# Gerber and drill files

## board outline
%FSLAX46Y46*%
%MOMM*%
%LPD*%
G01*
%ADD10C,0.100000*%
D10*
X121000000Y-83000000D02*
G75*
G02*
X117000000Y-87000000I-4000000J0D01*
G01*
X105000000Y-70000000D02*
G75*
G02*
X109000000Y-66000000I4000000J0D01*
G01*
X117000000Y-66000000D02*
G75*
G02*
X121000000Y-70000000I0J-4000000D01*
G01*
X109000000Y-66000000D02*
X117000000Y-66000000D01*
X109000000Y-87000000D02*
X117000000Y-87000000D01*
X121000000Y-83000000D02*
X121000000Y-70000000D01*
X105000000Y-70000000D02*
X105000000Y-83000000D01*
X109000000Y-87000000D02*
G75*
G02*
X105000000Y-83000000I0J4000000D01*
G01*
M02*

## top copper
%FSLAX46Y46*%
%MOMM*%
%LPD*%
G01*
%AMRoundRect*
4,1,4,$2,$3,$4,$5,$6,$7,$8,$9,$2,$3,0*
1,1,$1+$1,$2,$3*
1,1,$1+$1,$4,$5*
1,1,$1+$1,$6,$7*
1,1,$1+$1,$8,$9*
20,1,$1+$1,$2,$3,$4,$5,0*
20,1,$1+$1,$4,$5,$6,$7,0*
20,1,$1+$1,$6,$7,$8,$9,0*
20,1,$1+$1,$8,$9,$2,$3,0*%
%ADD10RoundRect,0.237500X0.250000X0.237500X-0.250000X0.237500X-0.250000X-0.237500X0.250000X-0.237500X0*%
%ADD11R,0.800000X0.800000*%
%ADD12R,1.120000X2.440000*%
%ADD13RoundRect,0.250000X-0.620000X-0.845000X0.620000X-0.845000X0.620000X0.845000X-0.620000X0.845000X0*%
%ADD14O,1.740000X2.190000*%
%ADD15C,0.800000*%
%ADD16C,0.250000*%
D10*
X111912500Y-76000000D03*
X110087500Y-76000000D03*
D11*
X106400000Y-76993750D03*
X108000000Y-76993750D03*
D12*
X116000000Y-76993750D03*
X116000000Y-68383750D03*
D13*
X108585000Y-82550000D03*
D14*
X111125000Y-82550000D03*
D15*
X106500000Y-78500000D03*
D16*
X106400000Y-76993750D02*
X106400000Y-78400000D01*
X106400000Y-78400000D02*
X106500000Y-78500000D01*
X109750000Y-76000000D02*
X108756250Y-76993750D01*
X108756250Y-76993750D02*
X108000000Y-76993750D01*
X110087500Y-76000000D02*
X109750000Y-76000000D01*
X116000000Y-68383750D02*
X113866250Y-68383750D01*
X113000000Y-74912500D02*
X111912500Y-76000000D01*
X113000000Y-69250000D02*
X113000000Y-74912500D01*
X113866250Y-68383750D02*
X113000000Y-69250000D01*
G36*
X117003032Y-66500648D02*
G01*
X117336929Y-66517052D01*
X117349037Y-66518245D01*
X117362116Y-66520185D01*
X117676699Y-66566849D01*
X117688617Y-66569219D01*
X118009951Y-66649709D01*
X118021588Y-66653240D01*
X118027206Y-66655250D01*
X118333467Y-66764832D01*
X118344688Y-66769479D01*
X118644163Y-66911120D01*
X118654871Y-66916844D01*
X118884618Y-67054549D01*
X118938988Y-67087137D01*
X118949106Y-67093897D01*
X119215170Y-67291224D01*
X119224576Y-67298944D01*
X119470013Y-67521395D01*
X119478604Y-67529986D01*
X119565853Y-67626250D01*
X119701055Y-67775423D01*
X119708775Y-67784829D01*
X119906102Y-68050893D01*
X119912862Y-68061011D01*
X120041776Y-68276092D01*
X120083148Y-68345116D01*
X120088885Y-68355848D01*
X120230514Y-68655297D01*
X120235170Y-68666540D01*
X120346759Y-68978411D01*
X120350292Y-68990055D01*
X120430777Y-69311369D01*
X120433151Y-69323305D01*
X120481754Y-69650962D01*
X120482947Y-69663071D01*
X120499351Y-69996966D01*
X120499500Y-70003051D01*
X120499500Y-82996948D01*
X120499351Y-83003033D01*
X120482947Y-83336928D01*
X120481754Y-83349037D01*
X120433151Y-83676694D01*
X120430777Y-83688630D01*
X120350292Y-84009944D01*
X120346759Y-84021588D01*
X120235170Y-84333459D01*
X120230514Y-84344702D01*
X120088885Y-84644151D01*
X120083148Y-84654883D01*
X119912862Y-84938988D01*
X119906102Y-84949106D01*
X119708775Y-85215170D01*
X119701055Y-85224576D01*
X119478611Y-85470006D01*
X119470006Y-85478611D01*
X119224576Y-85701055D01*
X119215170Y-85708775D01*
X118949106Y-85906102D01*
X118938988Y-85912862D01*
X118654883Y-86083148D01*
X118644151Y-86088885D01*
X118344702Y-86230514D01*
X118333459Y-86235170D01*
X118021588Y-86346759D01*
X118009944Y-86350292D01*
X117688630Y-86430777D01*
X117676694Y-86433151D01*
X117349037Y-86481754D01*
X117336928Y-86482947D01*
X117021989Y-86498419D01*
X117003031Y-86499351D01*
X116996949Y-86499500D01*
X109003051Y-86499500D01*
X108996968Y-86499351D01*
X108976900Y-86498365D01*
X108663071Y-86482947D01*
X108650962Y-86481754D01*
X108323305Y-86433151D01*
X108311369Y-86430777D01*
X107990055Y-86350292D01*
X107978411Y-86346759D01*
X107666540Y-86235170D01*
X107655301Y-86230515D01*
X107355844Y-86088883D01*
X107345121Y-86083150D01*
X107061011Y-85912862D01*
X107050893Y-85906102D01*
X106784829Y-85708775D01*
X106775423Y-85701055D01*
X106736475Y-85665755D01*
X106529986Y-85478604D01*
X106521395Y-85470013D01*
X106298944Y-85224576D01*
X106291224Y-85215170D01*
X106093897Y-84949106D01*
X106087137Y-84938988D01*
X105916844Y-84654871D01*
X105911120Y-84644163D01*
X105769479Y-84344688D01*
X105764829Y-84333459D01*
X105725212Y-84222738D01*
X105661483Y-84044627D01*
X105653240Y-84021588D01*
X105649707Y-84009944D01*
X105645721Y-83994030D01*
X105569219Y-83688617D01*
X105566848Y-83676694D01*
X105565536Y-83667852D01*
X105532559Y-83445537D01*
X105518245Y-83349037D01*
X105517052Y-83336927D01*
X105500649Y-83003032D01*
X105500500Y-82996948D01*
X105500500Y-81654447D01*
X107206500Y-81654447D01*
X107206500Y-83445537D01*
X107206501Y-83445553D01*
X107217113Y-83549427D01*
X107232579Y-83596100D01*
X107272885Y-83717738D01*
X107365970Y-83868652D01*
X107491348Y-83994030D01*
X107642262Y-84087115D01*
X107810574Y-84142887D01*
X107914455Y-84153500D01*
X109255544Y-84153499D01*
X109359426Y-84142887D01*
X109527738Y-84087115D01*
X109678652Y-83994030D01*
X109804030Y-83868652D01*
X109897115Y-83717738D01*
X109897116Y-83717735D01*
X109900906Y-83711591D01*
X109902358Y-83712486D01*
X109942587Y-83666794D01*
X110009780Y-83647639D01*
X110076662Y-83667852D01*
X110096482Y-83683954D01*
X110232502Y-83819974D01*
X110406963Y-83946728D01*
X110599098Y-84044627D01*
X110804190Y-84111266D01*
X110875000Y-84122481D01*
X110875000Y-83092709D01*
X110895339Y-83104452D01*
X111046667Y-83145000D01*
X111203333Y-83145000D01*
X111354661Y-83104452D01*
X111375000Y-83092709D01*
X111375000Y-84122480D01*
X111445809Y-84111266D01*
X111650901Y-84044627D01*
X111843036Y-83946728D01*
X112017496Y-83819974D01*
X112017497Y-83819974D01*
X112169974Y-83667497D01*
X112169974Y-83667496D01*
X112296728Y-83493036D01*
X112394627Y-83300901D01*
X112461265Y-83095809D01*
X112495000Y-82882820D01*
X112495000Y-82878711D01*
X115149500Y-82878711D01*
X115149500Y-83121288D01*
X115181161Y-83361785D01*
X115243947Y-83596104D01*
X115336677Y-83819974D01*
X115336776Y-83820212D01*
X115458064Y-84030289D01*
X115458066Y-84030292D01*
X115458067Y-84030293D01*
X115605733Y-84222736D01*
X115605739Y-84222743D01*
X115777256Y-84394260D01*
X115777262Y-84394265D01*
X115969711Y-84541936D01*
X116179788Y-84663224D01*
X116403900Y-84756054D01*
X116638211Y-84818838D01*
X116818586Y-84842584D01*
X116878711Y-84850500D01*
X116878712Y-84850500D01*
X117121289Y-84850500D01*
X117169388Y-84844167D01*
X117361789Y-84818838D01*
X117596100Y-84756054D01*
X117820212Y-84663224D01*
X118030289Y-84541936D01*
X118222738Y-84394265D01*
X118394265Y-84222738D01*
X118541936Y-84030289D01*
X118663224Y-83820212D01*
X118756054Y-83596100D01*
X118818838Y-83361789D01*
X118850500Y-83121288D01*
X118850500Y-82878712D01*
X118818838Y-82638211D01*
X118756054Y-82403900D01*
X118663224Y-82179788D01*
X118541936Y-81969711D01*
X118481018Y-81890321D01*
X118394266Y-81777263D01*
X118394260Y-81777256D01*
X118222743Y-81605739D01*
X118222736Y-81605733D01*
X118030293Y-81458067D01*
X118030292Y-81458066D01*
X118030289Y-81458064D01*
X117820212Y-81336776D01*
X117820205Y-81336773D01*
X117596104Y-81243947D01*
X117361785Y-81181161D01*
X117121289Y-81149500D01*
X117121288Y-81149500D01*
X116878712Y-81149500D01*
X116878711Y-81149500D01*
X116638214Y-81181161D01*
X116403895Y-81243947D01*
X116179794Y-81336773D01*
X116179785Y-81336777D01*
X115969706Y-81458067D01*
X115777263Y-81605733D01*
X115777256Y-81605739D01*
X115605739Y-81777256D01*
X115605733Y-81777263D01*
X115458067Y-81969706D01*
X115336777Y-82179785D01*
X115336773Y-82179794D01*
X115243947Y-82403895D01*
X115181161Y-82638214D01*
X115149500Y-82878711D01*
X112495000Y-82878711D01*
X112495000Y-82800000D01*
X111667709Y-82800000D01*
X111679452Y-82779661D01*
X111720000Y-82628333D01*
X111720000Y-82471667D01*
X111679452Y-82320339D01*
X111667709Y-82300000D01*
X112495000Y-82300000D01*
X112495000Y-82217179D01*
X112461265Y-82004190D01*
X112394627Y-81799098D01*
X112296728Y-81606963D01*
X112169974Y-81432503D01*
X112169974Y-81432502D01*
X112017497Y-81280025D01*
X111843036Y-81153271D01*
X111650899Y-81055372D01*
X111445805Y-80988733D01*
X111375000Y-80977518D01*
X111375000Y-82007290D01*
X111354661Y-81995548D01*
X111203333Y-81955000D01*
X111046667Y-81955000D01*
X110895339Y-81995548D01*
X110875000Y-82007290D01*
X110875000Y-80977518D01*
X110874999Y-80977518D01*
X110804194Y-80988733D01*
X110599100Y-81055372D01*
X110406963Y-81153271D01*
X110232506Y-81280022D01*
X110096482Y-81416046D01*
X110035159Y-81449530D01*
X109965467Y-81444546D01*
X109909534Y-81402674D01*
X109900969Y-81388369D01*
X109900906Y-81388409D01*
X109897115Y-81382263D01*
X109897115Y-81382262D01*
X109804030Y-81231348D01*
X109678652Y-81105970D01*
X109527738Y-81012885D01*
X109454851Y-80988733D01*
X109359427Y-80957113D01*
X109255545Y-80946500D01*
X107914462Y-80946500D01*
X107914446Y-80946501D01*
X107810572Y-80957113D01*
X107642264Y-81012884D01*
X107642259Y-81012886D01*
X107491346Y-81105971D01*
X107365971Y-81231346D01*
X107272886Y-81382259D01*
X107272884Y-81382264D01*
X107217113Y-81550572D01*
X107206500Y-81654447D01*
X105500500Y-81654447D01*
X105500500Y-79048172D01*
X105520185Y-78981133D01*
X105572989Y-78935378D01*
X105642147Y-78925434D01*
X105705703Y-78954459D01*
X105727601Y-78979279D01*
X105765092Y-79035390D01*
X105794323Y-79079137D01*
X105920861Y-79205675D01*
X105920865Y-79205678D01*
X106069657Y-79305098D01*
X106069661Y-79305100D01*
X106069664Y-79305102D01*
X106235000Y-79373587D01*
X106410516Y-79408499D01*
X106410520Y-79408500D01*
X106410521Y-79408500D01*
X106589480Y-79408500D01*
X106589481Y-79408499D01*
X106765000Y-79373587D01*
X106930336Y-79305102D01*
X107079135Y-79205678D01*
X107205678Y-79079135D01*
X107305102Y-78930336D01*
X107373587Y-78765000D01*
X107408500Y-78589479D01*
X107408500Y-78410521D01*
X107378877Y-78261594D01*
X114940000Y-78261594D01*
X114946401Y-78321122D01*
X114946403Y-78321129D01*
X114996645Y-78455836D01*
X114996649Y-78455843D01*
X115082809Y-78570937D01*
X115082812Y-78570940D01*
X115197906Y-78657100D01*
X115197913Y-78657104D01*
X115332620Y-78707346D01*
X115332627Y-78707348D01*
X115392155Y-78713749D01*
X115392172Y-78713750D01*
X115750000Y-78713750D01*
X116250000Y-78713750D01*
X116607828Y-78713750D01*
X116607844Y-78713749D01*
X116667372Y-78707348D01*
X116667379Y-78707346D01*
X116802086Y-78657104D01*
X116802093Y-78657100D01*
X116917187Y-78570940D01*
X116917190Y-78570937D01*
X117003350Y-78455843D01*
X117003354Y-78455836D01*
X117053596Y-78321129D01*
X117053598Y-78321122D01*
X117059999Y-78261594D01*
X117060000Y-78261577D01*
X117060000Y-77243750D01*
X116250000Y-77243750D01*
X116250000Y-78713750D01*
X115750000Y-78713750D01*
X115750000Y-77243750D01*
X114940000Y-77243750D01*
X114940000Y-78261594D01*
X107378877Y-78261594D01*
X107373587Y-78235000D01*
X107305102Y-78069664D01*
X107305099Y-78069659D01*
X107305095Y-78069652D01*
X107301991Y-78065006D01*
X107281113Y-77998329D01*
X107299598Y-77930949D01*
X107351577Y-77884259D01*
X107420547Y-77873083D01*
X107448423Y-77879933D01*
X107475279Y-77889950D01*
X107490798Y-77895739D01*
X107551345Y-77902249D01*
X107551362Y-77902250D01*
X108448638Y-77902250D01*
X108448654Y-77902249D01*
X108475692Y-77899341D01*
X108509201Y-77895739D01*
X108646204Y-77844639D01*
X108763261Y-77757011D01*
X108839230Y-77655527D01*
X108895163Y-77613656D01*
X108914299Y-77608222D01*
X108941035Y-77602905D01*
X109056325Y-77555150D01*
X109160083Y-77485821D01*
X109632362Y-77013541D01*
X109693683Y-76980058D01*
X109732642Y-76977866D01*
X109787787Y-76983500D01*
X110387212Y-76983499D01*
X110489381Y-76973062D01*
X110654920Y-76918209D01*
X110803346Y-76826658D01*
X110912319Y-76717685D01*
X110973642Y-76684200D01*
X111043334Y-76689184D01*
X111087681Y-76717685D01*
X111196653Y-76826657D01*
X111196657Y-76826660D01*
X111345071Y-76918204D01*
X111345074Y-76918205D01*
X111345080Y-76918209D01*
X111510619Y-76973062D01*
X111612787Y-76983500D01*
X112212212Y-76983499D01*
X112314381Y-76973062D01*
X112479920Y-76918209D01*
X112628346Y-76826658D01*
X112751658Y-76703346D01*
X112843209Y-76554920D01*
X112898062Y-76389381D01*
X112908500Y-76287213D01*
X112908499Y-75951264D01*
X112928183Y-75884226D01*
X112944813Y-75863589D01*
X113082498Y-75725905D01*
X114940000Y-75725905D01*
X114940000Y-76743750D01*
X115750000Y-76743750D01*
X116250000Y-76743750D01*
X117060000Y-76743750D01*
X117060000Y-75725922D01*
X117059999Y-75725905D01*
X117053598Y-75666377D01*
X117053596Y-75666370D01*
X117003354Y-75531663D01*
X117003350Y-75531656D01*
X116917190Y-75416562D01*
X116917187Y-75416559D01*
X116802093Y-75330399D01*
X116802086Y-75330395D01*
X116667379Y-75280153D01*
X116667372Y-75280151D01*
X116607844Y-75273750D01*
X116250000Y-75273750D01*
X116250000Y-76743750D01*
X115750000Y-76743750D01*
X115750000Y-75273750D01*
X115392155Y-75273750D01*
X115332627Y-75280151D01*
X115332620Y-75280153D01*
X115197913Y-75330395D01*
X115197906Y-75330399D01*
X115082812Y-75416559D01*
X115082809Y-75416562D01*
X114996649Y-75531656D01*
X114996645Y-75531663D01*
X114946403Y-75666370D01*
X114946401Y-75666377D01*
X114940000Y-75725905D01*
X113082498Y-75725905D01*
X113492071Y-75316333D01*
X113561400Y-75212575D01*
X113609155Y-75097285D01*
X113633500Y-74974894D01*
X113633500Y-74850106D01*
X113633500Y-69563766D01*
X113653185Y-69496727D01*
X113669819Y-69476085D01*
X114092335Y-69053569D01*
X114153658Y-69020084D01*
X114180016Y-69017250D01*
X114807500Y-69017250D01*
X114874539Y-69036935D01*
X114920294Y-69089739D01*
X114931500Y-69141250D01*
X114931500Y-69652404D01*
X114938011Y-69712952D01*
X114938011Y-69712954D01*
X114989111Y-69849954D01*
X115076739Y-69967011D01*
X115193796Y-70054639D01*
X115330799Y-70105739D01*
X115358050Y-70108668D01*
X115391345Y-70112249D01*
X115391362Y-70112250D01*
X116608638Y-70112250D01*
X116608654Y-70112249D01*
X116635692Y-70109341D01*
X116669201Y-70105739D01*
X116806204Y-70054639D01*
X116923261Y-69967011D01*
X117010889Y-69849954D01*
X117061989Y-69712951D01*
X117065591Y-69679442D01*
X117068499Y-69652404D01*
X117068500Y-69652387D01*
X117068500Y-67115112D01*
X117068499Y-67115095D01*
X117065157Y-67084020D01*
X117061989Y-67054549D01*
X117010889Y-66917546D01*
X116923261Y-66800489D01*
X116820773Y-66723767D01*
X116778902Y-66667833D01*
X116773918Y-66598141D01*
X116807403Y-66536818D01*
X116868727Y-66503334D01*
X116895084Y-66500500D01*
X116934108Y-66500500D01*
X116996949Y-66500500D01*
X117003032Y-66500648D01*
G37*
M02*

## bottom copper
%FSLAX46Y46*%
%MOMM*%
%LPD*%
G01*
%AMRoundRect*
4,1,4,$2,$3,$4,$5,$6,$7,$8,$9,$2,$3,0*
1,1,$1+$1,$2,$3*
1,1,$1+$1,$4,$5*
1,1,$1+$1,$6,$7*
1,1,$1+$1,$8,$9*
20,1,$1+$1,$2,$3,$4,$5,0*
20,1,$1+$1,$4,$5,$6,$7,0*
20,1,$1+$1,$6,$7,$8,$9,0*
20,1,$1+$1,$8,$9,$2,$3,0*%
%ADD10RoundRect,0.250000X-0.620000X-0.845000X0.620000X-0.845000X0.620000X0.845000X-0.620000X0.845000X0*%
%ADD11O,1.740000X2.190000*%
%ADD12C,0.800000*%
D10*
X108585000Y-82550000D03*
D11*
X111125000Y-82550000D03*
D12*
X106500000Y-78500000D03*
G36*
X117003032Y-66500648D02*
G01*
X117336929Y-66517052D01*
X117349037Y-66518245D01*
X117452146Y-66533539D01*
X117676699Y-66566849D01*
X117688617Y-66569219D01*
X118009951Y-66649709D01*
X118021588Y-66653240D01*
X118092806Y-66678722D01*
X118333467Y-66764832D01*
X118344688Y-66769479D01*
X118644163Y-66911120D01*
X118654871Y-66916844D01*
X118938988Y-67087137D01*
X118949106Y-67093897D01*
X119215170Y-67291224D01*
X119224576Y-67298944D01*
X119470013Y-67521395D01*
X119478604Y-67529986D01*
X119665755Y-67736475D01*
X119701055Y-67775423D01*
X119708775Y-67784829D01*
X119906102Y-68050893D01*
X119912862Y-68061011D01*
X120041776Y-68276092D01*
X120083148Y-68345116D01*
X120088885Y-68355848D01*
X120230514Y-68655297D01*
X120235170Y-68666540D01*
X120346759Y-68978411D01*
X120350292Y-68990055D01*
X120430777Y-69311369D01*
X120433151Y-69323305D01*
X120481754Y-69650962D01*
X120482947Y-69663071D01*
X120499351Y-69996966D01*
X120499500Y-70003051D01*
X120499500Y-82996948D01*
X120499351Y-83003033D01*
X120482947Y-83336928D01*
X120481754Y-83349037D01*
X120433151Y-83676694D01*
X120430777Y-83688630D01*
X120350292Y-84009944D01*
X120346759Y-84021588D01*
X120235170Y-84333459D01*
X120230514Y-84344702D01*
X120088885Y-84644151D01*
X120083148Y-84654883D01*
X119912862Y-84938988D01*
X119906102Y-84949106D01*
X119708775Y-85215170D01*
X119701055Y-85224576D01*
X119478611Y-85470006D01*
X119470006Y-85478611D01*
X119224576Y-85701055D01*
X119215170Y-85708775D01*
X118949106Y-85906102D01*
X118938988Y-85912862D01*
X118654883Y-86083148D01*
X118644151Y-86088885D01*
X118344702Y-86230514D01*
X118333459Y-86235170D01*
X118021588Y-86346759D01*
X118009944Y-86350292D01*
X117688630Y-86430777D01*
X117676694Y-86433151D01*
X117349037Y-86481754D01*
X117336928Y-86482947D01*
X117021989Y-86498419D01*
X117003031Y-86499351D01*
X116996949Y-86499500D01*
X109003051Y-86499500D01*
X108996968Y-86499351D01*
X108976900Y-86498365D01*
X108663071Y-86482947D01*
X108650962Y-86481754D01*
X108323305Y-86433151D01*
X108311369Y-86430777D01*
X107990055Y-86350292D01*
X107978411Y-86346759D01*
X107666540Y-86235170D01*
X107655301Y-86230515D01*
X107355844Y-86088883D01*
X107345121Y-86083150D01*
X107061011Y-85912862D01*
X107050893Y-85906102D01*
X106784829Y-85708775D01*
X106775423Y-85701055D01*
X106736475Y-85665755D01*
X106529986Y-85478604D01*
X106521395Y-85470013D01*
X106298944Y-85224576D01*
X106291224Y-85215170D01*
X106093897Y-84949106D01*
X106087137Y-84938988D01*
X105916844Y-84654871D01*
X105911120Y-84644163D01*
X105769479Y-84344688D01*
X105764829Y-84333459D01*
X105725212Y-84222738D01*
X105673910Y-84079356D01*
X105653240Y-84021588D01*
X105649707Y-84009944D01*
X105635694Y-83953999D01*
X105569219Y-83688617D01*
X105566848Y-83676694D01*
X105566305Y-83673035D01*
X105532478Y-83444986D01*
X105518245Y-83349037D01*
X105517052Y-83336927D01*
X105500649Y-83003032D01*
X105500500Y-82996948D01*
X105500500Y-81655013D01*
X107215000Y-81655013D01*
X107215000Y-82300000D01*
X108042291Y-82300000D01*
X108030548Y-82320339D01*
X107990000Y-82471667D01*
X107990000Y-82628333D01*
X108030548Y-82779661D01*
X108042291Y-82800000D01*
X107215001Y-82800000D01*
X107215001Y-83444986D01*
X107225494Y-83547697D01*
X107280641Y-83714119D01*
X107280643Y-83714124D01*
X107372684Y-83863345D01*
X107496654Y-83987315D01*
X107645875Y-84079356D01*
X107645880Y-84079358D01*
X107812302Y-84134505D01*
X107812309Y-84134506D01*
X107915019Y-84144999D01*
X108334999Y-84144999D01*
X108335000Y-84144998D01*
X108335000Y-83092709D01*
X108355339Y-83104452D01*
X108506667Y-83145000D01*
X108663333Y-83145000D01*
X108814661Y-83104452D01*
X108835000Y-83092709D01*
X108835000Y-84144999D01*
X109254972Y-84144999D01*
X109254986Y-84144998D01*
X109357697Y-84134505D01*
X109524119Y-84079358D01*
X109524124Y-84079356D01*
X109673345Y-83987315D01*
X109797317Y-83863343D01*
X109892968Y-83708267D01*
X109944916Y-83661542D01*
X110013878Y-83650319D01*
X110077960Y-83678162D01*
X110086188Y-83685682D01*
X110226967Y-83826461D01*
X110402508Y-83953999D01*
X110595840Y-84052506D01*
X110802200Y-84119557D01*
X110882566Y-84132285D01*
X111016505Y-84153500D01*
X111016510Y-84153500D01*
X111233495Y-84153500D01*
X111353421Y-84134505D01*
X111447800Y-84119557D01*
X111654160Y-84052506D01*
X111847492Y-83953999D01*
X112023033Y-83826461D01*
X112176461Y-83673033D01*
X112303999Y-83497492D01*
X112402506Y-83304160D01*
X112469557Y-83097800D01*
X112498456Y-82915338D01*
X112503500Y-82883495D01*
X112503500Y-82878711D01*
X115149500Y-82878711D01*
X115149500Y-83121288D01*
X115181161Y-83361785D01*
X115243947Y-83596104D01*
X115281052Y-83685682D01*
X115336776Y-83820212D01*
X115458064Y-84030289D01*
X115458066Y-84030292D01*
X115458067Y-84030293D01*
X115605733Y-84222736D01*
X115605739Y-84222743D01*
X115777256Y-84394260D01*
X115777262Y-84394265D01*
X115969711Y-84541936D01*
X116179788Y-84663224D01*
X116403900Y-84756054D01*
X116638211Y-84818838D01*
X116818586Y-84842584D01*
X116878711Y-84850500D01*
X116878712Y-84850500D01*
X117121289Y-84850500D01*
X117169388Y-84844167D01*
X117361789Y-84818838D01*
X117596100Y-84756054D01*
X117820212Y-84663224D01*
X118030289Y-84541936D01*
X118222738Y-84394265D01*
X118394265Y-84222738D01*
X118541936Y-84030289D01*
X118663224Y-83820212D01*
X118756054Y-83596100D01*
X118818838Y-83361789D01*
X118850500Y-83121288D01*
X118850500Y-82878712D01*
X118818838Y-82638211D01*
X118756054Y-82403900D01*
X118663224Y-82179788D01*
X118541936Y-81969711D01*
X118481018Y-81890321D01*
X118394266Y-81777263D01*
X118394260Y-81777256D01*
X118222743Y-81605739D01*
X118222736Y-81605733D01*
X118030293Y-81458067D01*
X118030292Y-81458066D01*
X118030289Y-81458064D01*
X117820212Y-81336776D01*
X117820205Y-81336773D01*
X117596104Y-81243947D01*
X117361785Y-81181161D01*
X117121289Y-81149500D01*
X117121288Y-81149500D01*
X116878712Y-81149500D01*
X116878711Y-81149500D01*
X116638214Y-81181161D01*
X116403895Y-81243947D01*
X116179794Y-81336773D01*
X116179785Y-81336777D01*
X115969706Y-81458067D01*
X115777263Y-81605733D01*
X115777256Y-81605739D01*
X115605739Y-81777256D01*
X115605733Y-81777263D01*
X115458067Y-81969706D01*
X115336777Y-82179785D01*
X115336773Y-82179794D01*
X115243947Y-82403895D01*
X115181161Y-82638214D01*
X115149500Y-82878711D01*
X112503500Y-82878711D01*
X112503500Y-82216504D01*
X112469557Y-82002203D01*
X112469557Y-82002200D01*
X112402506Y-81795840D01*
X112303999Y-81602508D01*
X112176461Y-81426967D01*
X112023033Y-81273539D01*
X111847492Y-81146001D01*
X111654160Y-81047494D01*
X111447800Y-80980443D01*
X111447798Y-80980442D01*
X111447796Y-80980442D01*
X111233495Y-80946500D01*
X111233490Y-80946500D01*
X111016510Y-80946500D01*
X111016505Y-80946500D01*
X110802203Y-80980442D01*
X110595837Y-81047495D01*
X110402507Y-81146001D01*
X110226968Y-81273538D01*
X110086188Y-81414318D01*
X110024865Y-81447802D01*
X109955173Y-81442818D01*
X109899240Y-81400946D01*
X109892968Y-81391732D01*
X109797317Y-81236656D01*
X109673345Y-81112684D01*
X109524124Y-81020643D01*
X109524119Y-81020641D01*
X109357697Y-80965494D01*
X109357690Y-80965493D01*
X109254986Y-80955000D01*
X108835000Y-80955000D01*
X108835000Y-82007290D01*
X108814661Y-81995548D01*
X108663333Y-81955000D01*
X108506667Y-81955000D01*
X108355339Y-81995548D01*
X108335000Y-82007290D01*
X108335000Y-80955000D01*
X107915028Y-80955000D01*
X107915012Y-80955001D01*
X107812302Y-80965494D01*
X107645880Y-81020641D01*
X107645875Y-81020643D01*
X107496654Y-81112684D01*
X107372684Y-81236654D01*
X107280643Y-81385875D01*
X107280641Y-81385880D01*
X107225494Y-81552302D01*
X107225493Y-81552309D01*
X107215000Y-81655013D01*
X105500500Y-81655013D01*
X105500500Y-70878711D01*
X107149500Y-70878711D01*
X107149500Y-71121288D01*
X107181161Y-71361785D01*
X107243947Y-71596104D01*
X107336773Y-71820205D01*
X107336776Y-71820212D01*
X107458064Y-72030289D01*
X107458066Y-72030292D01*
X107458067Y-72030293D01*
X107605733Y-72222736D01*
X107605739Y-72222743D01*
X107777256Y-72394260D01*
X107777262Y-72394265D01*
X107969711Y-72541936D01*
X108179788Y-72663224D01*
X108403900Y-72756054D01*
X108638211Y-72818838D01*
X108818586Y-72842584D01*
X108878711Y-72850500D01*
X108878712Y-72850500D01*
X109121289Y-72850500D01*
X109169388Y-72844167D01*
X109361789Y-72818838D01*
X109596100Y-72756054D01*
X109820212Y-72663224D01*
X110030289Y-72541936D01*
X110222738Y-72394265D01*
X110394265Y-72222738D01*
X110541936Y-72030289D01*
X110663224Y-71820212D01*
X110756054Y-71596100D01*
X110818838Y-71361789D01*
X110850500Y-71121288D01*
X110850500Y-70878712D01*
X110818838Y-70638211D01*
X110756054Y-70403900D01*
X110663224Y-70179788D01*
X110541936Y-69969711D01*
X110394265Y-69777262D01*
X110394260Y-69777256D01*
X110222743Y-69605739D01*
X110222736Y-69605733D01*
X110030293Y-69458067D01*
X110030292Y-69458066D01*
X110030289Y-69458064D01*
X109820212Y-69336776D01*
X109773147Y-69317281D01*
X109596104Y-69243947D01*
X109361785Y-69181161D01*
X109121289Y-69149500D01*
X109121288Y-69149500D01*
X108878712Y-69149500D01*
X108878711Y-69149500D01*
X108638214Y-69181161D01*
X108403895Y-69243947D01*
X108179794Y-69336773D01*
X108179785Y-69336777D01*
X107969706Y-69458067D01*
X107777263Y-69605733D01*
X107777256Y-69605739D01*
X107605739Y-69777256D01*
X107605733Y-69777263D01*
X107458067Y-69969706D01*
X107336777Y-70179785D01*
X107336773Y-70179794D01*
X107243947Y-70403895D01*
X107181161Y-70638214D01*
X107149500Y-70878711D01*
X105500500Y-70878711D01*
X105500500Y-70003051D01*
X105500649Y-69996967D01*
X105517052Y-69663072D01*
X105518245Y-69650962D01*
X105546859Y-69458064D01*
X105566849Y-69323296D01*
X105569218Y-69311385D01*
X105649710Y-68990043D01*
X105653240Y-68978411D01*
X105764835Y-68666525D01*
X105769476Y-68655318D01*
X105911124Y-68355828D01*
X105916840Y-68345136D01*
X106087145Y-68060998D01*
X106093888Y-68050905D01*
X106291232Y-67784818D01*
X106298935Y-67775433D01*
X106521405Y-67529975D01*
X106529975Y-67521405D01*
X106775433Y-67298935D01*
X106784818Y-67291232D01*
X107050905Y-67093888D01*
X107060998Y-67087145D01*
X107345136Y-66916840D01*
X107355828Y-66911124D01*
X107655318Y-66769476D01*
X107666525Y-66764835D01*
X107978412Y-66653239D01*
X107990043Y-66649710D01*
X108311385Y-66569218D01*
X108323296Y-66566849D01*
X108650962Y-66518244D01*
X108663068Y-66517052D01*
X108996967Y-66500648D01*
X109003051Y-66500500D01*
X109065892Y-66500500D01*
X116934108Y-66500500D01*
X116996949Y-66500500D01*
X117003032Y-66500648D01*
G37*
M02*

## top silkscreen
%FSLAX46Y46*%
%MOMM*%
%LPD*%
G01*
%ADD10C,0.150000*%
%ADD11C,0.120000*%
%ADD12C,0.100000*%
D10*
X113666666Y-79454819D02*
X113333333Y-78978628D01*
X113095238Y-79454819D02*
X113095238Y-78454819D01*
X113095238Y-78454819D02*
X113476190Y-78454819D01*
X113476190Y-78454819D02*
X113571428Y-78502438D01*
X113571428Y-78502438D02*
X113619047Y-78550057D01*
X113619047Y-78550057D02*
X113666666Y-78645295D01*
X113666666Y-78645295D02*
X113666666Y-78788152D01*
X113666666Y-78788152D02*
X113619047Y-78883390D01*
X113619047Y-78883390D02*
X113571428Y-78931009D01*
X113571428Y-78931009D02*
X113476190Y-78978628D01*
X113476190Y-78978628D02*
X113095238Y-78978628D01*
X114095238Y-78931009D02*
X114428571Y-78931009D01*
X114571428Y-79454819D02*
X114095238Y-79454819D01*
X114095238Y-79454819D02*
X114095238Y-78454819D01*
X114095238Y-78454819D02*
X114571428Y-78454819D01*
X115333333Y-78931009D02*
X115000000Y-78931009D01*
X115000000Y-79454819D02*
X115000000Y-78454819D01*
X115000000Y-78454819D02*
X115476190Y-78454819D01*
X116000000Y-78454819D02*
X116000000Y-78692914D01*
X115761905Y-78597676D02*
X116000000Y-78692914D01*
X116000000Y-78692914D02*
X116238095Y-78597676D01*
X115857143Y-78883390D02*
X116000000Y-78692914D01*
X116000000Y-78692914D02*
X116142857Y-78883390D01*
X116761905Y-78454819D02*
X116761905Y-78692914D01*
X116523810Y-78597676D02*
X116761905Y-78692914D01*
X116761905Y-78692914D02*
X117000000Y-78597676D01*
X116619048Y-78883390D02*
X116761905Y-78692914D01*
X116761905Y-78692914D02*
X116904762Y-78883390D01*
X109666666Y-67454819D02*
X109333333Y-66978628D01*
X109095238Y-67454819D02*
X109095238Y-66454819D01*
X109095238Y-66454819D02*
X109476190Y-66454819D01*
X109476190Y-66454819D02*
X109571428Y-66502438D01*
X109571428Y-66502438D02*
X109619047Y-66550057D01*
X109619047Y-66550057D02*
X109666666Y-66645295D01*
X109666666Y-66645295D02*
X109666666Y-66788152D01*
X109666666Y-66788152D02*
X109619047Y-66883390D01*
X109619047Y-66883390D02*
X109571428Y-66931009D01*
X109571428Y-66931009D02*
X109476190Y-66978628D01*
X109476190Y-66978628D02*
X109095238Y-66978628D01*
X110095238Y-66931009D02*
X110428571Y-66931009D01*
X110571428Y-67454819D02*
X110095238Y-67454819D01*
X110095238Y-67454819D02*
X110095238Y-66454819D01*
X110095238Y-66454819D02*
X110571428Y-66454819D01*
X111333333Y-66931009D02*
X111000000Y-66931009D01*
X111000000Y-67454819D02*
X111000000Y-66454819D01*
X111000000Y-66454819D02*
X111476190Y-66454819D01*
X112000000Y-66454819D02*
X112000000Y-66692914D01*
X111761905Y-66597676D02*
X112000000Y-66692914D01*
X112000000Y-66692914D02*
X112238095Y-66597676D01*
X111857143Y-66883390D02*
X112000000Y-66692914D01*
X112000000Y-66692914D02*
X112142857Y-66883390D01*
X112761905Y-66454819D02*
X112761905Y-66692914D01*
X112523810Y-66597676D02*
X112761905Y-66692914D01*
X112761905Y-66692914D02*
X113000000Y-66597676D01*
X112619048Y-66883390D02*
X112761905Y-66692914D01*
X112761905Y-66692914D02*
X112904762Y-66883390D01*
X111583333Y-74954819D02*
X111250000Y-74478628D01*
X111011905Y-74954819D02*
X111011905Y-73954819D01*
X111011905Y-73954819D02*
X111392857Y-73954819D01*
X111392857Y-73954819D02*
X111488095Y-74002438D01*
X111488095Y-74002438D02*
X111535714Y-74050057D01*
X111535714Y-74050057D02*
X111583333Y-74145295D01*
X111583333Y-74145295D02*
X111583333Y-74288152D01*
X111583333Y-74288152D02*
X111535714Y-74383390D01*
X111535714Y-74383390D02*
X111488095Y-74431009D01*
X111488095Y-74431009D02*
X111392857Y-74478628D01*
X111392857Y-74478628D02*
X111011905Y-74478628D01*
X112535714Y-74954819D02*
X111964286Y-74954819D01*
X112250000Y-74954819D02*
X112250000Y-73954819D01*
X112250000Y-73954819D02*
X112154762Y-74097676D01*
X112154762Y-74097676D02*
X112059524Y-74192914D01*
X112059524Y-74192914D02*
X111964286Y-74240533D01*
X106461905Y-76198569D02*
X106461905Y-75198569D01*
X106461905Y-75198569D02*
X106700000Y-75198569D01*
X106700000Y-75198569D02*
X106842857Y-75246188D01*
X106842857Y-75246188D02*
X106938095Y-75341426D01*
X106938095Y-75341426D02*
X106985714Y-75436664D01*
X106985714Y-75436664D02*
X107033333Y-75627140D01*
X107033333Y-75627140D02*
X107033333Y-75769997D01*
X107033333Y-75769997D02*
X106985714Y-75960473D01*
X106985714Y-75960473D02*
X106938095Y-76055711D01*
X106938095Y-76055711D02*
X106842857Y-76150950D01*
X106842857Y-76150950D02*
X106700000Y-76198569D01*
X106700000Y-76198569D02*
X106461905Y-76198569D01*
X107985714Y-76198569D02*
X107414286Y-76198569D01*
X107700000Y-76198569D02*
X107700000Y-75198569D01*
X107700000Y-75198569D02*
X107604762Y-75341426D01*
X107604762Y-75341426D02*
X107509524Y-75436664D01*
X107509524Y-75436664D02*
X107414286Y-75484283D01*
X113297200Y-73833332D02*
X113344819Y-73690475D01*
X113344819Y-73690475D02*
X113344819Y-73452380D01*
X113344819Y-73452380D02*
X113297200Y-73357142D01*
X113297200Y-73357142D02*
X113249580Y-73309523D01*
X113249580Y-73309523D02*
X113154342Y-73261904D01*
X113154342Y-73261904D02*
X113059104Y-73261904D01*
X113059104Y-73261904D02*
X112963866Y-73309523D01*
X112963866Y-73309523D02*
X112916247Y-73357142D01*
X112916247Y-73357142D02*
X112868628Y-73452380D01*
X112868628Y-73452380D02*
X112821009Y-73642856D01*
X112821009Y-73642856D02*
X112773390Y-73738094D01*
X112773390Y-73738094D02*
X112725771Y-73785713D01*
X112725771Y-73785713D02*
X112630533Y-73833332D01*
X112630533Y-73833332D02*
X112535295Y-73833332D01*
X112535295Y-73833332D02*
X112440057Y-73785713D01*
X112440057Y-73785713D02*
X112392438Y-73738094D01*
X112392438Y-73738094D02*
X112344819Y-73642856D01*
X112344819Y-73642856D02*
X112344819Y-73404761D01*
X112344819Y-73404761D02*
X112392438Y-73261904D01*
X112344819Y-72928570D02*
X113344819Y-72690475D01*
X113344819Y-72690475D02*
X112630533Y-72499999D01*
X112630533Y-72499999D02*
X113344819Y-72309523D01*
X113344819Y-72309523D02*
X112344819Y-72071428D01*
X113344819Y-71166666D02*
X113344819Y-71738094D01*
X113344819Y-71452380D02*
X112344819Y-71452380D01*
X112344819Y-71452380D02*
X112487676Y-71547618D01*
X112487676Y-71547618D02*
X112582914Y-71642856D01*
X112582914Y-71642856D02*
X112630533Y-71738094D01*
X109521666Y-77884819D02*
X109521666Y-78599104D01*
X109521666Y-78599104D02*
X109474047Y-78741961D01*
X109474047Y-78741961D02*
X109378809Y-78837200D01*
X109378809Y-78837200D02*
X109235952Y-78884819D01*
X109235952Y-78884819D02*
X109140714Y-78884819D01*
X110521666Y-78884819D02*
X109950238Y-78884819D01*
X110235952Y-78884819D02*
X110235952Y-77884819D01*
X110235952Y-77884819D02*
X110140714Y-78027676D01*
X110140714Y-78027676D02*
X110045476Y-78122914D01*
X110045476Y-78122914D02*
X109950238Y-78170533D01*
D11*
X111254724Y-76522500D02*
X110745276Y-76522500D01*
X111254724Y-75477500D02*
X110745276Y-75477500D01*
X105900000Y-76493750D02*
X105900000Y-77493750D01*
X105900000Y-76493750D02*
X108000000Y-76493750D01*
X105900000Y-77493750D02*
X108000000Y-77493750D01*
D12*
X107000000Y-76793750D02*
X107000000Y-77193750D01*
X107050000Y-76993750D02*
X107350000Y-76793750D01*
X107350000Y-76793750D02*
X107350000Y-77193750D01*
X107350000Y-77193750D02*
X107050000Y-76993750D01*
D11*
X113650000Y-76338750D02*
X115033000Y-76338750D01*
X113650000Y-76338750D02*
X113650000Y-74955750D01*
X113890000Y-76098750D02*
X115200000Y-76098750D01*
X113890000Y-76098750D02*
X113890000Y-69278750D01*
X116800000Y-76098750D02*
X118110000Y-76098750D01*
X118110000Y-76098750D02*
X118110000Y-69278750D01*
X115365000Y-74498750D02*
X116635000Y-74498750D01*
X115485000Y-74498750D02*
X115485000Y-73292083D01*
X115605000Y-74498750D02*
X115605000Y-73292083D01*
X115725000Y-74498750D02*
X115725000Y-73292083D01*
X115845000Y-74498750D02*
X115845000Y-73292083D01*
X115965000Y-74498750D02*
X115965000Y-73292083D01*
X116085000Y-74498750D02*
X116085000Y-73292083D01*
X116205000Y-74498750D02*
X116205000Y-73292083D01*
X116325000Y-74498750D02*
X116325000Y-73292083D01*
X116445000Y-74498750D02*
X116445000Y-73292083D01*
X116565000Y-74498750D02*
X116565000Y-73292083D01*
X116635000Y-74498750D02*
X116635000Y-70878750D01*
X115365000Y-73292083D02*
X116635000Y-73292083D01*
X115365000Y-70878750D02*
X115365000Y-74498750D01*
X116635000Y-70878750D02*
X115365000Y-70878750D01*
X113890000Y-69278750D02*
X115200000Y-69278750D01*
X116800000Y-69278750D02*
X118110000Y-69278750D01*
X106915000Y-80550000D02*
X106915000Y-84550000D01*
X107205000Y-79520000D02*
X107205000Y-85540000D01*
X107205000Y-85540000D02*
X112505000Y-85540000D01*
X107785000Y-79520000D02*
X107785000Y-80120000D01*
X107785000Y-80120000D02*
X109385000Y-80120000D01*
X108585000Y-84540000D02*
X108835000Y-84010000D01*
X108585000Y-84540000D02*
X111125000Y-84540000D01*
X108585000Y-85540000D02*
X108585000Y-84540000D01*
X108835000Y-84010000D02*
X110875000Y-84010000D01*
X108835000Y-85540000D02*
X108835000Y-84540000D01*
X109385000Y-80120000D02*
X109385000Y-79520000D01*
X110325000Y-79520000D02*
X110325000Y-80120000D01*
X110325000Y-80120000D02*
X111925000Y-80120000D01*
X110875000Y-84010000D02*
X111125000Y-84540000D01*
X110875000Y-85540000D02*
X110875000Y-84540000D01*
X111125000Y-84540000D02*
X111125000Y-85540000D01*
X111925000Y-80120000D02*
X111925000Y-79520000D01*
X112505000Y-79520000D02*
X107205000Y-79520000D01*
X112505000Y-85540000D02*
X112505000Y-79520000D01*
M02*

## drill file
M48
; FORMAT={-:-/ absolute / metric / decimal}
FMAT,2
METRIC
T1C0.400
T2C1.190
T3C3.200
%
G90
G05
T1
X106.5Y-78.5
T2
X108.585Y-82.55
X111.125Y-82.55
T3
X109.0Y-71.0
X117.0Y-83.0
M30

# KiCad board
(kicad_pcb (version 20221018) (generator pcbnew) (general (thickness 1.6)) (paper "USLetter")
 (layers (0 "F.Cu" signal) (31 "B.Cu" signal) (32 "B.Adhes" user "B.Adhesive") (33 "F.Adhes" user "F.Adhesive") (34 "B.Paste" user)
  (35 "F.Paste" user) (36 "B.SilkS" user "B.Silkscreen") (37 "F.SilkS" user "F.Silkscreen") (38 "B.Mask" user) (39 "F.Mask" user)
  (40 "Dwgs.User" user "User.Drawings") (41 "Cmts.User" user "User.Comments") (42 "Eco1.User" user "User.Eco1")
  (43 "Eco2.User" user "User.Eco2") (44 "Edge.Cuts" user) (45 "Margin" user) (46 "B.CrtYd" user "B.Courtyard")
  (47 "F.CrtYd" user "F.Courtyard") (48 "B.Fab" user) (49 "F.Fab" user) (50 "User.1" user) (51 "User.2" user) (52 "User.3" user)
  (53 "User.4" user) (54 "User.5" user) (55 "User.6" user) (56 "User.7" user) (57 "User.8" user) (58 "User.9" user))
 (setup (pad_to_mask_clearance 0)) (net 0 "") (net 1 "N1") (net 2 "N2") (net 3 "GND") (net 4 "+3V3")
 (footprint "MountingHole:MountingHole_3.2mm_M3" (layer "F.Cu") (at 117 83)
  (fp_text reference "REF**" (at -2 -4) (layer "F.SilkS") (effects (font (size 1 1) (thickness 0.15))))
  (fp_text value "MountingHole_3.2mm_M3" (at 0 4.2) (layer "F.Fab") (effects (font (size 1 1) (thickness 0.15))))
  (pad "" np_thru_hole circle (at 0 0) (size 3.2 3.2) (drill 3.2) (layers "*.Cu" "*.Mask")))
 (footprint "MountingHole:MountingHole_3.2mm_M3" (layer "F.Cu") (at 109 71)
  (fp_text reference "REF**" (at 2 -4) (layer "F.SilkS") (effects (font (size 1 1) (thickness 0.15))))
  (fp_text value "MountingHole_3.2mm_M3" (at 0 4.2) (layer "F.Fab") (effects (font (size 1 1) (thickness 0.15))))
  (pad "" np_thru_hole circle (at 0 0) (size 3.2 3.2) (drill 3.2) (layers "*.Cu" "*.Mask")))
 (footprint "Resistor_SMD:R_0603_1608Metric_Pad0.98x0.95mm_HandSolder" (layer "F.Cu") (at 111 76 180)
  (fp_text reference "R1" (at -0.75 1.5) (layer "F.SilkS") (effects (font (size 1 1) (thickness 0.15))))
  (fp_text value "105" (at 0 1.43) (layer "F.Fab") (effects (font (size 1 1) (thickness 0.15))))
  (fp_line (start -0.254724 -0.5225) (end 0.254724 -0.5225) (stroke (width 0.12) (type solid)) (layer "F.SilkS"))
  (fp_line (start -0.254724 0.5225) (end 0.254724 0.5225) (stroke (width 0.12) (type solid)) (layer "F.SilkS"))
  (pad "1" smd roundrect (at -0.9125 0 180) (size 0.975 0.95) (layers "F.Cu" "F.Paste" "F.Mask") (roundrect_rratio 0.25) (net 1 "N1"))
  (pad "2" smd roundrect (at 0.9125 0 180) (size 0.975 0.95) (layers "F.Cu" "F.Paste" "F.Mask") (roundrect_rratio 0.25) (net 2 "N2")))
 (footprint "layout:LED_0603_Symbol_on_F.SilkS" (layer "F.Cu") (at 107.2 76.99375)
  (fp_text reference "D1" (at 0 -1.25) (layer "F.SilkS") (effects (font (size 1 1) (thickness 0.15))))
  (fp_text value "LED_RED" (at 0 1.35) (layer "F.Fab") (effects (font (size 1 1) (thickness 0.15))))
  (fp_line (start -1.3 -0.5) (end -1.3 0.5) (stroke (width 0.12) (type solid)) (layer "F.SilkS"))
  (fp_line (start -1.3 -0.5) (end 0.8 -0.5) (stroke (width 0.12) (type solid)) (layer "F.SilkS"))
  (fp_line (start -1.3 0.5) (end 0.8 0.5) (stroke (width 0.12) (type solid)) (layer "F.SilkS"))
  (fp_line (start -0.2 -0.2) (end -0.2 0.2) (stroke (width 0.1) (type solid)) (layer "F.SilkS"))
  (fp_line (start -0.15 0) (end 0.15 -0.2) (stroke (width 0.1) (type solid)) (layer "F.SilkS"))
  (fp_line (start 0.15 -0.2) (end 0.15 0.2) (stroke (width 0.1) (type solid)) (layer "F.SilkS"))
  (fp_line (start 0.15 0.2) (end -0.15 0) (stroke (width 0.1) (type solid)) (layer "F.SilkS"))
  (pad "1" smd rect (at -0.8 0 180) (size 0.8 0.8) (layers "F.Cu" "F.Paste" "F.Mask") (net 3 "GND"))
  (pad "2" smd rect (at 0.8 0 180) (size 0.8 0.8) (layers "F.Cu" "F.Paste" "F.Mask") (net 2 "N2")))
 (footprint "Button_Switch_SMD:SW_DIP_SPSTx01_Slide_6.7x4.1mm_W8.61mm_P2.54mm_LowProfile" (layer "F.Cu") (at 116 72.68875 90)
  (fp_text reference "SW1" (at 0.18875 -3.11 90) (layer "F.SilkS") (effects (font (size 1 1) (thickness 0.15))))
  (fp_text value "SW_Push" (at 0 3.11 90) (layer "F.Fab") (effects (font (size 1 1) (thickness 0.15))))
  (fp_line (start -3.65 -2.35) (end -3.65 -0.967) (stroke (width 0.12) (type solid)) (layer "F.SilkS"))
  (fp_line (start -3.65 -2.35) (end -2.267 -2.35) (stroke (width 0.12) (type solid)) (layer "F.SilkS"))
  (fp_line (start -3.41 -2.11) (end -3.41 -0.8) (stroke (width 0.12) (type solid)) (layer "F.SilkS"))
  (fp_line (start -3.41 -2.11) (end 3.41 -2.11) (stroke (width 0.12) (type solid)) (layer "F.SilkS"))
  (fp_line (start -3.41 0.8) (end -3.41 2.11) (stroke (width 0.12) (type solid)) (layer "F.SilkS"))
  (fp_line (start -3.41 2.11) (end 3.41 2.11) (stroke (width 0.12) (type solid)) (layer "F.SilkS"))
  (fp_line (start -1.81 -0.635) (end -1.81 0.635) (stroke (width 0.12) (type solid)) (layer "F.SilkS"))
  (fp_line (start -1.81 -0.515) (end -0.603333 -0.515) (stroke (width 0.12) (type solid)) (layer "F.SilkS"))
  (fp_line (start -1.81 -0.395) (end -0.603333 -0.395) (stroke (width 0.12) (type solid)) (layer "F.SilkS"))
  (fp_line (start -1.81 -0.275) (end -0.603333 -0.275) (stroke (width 0.12) (type solid)) (layer "F.SilkS"))
  (fp_line (start -1.81 -0.155) (end -0.603333 -0.155) (stroke (width 0.12) (type solid)) (layer "F.SilkS"))
  (fp_line (start -1.81 -0.035) (end -0.603333 -0.035) (stroke (width 0.12) (type solid)) (layer "F.SilkS"))
  (fp_line (start -1.81 0.085) (end -0.603333 0.085) (stroke (width 0.12) (type solid)) (layer "F.SilkS"))
  (fp_line (start -1.81 0.205) (end -0.603333 0.205) (stroke (width 0.12) (type solid)) (layer "F.SilkS"))
  (fp_line (start -1.81 0.325) (end -0.603333 0.325) (stroke (width 0.12) (type solid)) (layer "F.SilkS"))
  (fp_line (start -1.81 0.445) (end -0.603333 0.445) (stroke (width 0.12) (type solid)) (layer "F.SilkS"))
  (fp_line (start -1.81 0.565) (end -0.603333 0.565) (stroke (width 0.12) (type solid)) (layer "F.SilkS"))
  (fp_line (start -1.81 0.635) (end 1.81 0.635) (stroke (width 0.12) (type solid)) (layer "F.SilkS"))
  (fp_line (start -0.603333 -0.635) (end -0.603333 0.635) (stroke (width 0.12) (type solid)) (layer "F.SilkS"))
  (fp_line (start 1.81 -0.635) (end -1.81 -0.635) (stroke (width 0.12) (type solid)) (layer "F.SilkS"))
  (fp_line (start 1.81 0.635) (end 1.81 -0.635) (stroke (width 0.12) (type solid)) (layer "F.SilkS"))
  (fp_line (start 3.41 -2.11) (end 3.41 -0.8) (stroke (width 0.12) (type solid)) (layer "F.SilkS"))
  (fp_line (start 3.41 0.8) (end 3.41 2.11) (stroke (width 0.12) (type solid)) (layer "F.SilkS"))
  (pad "1" smd rect (at -4.305 0 90) (size 2.44 1.12) (layers "F.Cu" "F.Paste" "F.Mask") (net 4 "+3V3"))
  (pad "2" smd rect (at 4.305 0 90) (size 2.44 1.12) (layers "F.Cu" "F.Paste" "F.Mask") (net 1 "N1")))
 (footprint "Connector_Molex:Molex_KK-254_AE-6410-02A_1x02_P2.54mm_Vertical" (layer "F.Cu") (at 108.585 82.55)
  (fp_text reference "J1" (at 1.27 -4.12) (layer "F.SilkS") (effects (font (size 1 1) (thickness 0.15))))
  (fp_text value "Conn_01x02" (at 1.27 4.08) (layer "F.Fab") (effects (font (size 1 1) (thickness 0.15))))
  (fp_line (start -1.67 -2) (end -1.67 2) (stroke (width 0.12) (type solid)) (layer "F.SilkS"))
  (fp_line (start -1.38 -3.03) (end -1.38 2.99) (stroke (width 0.12) (type solid)) (layer "F.SilkS"))
  (fp_line (start -1.38 2.99) (end 3.92 2.99) (stroke (width 0.12) (type solid)) (layer "F.SilkS"))
  (fp_line (start -0.8 -3.03) (end -0.8 -2.43) (stroke (width 0.12) (type solid)) (layer "F.SilkS"))
  (fp_line (start -0.8 -2.43) (end 0.8 -2.43) (stroke (width 0.12) (type solid)) (layer "F.SilkS"))
  (fp_line (start 0 1.99) (end 0.25 1.46) (stroke (width 0.12) (type solid)) (layer "F.SilkS"))
  (fp_line (start 0 1.99) (end 2.54 1.99) (stroke (width 0.12) (type solid)) (layer "F.SilkS"))
  (fp_line (start 0 2.99) (end 0 1.99) (stroke (width 0.12) (type solid)) (layer "F.SilkS"))
  (fp_line (start 0.25 1.46) (end 2.29 1.46) (stroke (width 0.12) (type solid)) (layer "F.SilkS"))
  (fp_line (start 0.25 2.99) (end 0.25 1.99) (stroke (width 0.12) (type solid)) (layer "F.SilkS"))
  (fp_line (start 0.8 -2.43) (end 0.8 -3.03) (stroke (width 0.12) (type solid)) (layer "F.SilkS"))
  (fp_line (start 1.74 -3.03) (end 1.74 -2.43) (stroke (width 0.12) (type solid)) (layer "F.SilkS"))
  (fp_line (start 1.74 -2.43) (end 3.34 -2.43) (stroke (width 0.12) (type solid)) (layer "F.SilkS"))
  (fp_line (start 2.29 1.46) (end 2.54 1.99) (stroke (width 0.12) (type solid)) (layer "F.SilkS"))
  (fp_line (start 2.29 2.99) (end 2.29 1.99) (stroke (width 0.12) (type solid)) (layer "F.SilkS"))
  (fp_line (start 2.54 1.99) (end 2.54 2.99) (stroke (width 0.12) (type solid)) (layer "F.SilkS"))
  (fp_line (start 3.34 -2.43) (end 3.34 -3.03) (stroke (width 0.12) (type solid)) (layer "F.SilkS"))
  (fp_line (start 3.92 -3.03) (end -1.38 -3.03) (stroke (width 0.12) (type solid)) (layer "F.SilkS"))
  (fp_line (start 3.92 2.99) (end 3.92 -3.03) (stroke (width 0.12) (type solid)) (layer "F.SilkS"))
  (pad "1" thru_hole roundrect (at 0 0) (size 1.74 2.19) (drill 1.19) (layers "*.Cu" "*.Mask") (roundrect_rratio 0.143678) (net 3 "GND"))
  (pad "2" thru_hole oval (at 2.54 0) (size 1.74 2.19) (drill 1.19) (layers "*.Cu" "*.Mask") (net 4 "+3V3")))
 (gr_arc (start 121 83) (mid 119.828427 85.828427) (end 117 87) (stroke (width 0.1) (type default)) (layer "Edge.Cuts"))
 (gr_arc (start 105 70) (mid 106.171573 67.171573) (end 109 66) (stroke (width 0.1) (type default)) (layer "Edge.Cuts"))
 (gr_arc (start 117 66) (mid 119.828427 67.171573) (end 121 70) (stroke (width 0.1) (type default)) (layer "Edge.Cuts"))
 (gr_line (start 109 66) (end 117 66) (stroke (width 0.1) (type default)) (layer "Edge.Cuts"))
 (gr_line (start 109 87) (end 117 87) (stroke (width 0.1) (type default)) (layer "Edge.Cuts"))
 (gr_line (start 121 83) (end 121 70) (stroke (width 0.1) (type default)) (layer "Edge.Cuts"))
 (gr_line (start 105 70) (end 105 83) (stroke (width 0.1) (type default)) (layer "Edge.Cuts"))
 (gr_arc (start 109 87) (mid 106.171573 85.828427) (end 105 83) (stroke (width 0.1) (type default)) (layer "Edge.Cuts"))
 (segment (start 106.4 76.99375) (end 106.4 78.4) (width 0.25) (layer "F.Cu") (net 3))
 (segment (start 106.4 78.4) (end 106.5 78.5) (width 0.25) (layer "F.Cu") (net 3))
 (via (at 106.5 78.5) (size 0.8) (drill 0.4) (layers "F.Cu" "B.Cu") (free) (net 3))
 (segment (start 109.75 76) (end 108.75625 76.99375) (width 0.25) (layer "F.Cu") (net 2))
 (segment (start 108.75625 76.99375) (end 108 76.99375) (width 0.25) (layer "F.Cu") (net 2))
 (segment (start 110.0875 76) (end 109.75 76) (width 0.25) (layer "F.Cu") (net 2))
 (segment (start 116 68.38375) (end 113.86625 68.38375) (width 0.25) (layer "F.Cu") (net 1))
 (segment (start 113 74.9125) (end 111.9125 76) (width 0.25) (layer "F.Cu") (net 1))
 (segment (start 113 69.25) (end 113 74.9125) (width 0.25) (layer "F.Cu") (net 1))
 (segment (start 113.86625 68.38375) (end 113 69.25) (width 0.25) (layer "F.Cu") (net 1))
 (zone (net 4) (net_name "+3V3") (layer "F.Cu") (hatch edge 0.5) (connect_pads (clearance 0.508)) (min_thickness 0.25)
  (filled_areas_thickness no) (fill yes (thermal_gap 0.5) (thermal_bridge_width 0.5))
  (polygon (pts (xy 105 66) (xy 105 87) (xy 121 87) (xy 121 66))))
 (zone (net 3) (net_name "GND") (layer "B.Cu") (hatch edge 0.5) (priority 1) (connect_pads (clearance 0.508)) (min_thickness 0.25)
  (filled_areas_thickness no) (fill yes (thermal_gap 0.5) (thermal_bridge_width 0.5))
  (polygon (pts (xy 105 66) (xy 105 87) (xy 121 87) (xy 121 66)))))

